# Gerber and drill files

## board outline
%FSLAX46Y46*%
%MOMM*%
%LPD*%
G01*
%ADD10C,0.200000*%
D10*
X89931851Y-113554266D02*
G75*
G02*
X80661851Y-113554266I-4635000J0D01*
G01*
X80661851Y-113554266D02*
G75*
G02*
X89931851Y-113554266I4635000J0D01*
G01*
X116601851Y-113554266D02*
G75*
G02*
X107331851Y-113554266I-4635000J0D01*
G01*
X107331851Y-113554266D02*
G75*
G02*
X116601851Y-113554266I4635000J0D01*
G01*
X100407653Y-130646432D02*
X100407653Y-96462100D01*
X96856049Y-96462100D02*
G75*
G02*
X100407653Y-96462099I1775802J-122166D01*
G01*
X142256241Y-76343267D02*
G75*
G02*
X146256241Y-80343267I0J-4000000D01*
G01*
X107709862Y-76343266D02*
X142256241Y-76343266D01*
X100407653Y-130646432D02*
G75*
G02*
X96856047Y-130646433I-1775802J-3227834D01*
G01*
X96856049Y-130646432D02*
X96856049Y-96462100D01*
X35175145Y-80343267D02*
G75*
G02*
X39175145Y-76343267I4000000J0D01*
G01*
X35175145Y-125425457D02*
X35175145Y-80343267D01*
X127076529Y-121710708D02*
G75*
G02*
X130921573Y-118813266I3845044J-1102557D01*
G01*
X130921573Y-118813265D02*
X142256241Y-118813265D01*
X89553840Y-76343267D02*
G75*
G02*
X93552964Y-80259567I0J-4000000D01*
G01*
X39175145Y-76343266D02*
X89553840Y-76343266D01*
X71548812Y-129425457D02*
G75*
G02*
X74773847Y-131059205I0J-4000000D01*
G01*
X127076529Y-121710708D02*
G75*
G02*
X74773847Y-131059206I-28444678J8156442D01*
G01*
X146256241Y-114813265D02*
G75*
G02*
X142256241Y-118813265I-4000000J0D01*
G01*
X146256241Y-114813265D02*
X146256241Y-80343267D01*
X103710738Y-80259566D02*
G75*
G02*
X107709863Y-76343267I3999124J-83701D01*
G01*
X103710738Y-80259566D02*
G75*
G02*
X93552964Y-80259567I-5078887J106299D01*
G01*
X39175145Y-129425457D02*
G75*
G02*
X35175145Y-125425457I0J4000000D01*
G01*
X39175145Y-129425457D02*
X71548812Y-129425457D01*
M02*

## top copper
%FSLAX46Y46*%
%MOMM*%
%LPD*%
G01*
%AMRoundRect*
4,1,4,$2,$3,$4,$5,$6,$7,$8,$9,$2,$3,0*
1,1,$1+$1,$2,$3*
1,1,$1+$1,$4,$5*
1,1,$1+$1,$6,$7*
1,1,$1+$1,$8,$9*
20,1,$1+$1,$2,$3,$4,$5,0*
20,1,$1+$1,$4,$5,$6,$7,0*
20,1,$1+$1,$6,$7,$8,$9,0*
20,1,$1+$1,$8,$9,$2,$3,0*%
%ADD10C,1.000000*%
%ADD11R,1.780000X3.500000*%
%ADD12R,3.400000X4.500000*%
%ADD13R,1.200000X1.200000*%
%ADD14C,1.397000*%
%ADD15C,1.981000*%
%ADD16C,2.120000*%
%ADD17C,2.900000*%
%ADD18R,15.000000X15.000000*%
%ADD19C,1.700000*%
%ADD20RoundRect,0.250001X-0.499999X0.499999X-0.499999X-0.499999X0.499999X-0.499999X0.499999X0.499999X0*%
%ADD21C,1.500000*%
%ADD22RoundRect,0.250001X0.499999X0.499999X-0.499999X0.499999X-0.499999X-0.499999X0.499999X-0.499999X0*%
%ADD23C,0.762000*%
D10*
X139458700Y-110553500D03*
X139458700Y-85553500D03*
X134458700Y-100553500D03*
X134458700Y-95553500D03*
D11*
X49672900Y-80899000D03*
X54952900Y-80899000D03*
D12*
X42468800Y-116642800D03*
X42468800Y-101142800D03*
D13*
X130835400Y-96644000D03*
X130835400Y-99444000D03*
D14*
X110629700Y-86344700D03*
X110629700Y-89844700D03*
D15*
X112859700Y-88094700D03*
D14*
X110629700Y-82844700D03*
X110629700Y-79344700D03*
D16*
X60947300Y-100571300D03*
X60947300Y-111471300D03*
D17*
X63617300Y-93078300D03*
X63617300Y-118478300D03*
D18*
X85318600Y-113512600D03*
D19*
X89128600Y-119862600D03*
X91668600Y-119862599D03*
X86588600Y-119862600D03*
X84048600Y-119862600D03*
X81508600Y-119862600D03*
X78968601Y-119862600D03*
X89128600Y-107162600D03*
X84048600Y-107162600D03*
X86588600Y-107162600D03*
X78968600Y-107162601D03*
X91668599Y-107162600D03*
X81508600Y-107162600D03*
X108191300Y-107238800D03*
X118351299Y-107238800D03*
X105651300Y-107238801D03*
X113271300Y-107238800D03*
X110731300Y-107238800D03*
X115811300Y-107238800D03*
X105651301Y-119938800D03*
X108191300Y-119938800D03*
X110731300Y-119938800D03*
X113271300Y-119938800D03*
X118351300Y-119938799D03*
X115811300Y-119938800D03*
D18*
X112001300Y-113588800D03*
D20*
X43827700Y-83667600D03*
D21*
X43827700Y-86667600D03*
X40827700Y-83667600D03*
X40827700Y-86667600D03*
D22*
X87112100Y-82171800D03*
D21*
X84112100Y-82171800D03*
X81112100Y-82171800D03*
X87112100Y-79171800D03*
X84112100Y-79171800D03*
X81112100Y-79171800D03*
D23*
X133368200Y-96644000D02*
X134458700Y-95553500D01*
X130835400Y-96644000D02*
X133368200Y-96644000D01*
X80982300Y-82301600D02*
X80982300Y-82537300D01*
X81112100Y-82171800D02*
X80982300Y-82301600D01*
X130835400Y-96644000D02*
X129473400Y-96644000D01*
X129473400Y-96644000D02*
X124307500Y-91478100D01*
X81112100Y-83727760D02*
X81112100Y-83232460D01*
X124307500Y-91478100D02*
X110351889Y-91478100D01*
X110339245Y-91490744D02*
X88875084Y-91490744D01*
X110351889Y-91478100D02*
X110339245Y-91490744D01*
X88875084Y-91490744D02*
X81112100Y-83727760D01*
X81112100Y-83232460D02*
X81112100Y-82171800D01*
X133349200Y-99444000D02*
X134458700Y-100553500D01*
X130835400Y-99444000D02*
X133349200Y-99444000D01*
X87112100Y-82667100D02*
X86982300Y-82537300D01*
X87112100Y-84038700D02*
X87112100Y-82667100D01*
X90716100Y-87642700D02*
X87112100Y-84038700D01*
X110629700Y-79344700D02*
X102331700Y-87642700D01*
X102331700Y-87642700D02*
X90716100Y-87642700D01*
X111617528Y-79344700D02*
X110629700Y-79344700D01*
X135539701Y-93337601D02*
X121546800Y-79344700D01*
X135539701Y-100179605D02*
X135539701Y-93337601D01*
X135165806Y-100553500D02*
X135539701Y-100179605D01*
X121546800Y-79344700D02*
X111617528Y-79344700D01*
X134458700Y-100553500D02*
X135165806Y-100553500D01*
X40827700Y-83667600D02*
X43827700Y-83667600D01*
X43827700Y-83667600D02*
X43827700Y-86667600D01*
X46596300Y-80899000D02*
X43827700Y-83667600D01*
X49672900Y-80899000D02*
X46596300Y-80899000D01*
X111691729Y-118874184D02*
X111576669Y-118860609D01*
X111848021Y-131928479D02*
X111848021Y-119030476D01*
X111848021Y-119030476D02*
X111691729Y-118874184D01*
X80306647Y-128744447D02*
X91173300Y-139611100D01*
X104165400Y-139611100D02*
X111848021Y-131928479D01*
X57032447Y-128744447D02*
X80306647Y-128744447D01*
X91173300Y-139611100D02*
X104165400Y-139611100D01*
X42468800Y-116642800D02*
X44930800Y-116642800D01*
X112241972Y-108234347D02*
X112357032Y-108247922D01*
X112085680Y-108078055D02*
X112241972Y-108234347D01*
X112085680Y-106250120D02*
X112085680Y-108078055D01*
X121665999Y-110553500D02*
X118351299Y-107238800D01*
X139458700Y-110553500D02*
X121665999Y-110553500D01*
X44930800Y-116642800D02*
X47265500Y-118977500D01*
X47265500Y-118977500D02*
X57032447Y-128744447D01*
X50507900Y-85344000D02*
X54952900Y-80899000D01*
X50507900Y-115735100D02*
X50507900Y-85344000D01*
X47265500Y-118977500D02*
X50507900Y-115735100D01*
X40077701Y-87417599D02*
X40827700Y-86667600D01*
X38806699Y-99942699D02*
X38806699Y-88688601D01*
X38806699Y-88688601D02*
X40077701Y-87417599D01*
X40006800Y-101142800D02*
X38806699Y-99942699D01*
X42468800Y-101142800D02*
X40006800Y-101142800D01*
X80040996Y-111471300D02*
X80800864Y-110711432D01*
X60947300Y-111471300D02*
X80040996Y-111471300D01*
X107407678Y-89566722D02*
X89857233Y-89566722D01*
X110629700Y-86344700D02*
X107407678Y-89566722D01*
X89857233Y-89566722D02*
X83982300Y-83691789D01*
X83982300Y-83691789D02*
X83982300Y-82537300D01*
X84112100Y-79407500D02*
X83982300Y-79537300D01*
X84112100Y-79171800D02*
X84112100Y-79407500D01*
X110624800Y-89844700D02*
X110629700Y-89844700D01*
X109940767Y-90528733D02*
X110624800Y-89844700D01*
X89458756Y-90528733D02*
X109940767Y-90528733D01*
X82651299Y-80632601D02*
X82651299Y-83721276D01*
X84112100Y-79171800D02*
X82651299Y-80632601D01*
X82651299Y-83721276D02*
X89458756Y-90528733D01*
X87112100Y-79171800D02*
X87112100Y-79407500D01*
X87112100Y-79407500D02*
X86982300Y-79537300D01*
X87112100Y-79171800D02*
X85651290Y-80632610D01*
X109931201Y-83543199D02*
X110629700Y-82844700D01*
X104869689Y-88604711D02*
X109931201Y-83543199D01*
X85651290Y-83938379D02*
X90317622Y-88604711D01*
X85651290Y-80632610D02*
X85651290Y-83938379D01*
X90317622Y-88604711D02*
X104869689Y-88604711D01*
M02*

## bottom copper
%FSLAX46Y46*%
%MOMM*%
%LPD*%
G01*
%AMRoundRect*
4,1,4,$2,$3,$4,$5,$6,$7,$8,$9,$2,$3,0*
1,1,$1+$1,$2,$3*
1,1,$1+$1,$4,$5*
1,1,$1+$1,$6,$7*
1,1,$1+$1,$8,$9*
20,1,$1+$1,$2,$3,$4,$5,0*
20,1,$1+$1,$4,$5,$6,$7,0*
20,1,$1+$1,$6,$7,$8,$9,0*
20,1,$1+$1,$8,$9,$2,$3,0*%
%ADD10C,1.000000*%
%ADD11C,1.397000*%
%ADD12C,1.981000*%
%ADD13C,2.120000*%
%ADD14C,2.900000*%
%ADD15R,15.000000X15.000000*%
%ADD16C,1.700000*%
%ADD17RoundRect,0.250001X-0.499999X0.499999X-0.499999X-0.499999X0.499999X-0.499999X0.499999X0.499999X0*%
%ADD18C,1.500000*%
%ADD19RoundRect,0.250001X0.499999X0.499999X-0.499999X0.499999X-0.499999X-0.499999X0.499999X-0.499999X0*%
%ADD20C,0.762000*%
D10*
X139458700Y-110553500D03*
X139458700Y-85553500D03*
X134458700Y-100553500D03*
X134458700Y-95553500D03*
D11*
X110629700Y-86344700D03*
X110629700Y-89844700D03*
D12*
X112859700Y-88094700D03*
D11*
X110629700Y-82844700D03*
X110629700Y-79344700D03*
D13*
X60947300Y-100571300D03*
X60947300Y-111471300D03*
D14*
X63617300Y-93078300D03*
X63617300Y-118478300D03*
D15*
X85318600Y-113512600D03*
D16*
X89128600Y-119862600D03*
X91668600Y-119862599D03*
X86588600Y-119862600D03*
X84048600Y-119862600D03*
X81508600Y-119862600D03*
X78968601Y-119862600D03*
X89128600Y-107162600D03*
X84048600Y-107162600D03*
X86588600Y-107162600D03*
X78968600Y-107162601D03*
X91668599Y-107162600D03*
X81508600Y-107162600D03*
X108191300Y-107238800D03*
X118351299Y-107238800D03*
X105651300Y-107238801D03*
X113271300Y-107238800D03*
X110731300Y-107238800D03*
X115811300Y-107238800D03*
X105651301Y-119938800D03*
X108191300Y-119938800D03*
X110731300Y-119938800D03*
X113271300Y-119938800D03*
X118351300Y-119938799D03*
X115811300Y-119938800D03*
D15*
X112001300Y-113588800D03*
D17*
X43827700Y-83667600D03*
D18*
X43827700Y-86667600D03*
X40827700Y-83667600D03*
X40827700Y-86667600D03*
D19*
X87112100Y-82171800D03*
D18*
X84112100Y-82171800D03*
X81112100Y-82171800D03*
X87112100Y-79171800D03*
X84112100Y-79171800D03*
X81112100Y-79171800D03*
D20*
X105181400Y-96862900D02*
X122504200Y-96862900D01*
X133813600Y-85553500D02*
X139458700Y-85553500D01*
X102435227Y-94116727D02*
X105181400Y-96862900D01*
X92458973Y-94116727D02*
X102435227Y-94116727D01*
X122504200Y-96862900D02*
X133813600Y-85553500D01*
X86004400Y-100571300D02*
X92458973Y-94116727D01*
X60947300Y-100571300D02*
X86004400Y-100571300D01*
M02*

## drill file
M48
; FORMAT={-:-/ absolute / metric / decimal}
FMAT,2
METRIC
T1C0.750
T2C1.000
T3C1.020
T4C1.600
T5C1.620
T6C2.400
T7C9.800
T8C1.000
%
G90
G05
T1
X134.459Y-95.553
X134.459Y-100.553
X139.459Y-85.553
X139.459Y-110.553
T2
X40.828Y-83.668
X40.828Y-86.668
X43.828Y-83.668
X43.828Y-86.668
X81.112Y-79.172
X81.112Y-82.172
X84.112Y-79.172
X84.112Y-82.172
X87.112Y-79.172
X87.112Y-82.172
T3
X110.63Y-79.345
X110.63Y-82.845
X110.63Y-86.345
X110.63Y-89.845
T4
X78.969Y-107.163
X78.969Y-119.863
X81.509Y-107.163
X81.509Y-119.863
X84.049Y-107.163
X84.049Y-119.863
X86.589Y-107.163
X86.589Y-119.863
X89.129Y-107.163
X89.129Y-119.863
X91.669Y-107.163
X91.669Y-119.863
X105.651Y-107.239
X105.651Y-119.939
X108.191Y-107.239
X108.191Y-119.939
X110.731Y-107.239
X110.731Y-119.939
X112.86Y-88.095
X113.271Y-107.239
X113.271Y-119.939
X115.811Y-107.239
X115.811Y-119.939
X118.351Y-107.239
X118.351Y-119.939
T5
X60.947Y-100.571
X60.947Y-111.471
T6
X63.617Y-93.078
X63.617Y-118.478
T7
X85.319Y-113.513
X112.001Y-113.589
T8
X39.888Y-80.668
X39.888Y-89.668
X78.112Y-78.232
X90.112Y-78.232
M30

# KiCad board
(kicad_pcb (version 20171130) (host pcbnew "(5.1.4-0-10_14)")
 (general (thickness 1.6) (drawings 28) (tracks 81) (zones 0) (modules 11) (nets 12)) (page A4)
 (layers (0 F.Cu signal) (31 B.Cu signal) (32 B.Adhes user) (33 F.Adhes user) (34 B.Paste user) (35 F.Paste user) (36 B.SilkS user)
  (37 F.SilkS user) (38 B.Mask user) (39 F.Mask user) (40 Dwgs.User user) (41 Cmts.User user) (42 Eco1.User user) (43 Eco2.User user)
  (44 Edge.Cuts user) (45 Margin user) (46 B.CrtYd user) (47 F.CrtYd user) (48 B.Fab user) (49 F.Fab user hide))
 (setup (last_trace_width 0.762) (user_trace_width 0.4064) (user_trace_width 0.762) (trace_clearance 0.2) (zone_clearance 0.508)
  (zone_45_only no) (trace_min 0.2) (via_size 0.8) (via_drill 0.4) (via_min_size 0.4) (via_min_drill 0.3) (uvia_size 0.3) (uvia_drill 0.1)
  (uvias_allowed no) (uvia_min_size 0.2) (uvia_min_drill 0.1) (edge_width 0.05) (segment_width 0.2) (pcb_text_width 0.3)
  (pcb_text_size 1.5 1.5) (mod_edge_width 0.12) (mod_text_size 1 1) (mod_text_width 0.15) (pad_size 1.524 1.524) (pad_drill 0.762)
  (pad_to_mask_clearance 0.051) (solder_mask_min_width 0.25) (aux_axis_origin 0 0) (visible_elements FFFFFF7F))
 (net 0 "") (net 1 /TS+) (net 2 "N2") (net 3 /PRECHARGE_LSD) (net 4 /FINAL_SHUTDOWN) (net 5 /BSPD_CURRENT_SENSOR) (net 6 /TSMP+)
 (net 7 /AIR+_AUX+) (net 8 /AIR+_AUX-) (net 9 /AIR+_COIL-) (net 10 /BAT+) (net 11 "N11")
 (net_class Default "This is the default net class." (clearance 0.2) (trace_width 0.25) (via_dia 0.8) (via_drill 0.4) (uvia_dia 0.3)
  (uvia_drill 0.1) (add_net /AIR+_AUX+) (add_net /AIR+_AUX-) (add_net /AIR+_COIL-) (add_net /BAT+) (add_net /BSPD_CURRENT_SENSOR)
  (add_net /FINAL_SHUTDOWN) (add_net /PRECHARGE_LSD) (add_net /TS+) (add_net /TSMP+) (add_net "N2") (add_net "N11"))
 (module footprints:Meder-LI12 (layer F.Cu) (at 139.4587 110.5535 90)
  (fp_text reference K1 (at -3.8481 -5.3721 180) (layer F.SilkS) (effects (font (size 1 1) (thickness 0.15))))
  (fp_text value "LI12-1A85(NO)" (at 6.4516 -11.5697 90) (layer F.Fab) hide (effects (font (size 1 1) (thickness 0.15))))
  (pad 1 thru_hole circle (at 0 0 90) (size 1 1) (drill 0.75) (layers *.Cu *.Mask) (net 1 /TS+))
  (pad 2 thru_hole circle (at 25 0 90) (size 1 1) (drill 0.75) (layers *.Cu *.Mask) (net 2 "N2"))
  (pad 3 thru_hole circle (at 10 -5 90) (size 1 1) (drill 0.75) (layers *.Cu *.Mask) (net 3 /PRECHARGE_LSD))
  (pad 4 thru_hole circle (at 15 -5 90) (size 1 1) (drill 0.75) (layers *.Cu *.Mask) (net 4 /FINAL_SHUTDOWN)))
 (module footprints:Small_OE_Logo (layer F.Cu) (at 84.9503 96.774)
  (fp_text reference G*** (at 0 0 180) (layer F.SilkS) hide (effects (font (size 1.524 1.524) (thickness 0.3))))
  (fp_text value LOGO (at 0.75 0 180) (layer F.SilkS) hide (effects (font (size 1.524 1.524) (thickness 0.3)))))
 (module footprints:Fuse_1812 (layer F.Cu) (at 54.9529 80.899 180)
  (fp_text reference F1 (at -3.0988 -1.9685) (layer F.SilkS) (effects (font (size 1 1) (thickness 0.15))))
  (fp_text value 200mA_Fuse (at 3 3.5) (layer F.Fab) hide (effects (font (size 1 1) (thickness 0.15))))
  (pad 2 smd rect (at 5.28 0 180) (size 1.78 3.5) (layers F.Cu F.Paste F.Mask) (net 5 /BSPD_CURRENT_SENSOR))
  (pad 1 smd rect (at 0 0 180) (size 1.78 3.5) (layers F.Cu F.Paste F.Mask) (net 1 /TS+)))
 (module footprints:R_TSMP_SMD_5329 (layer F.Cu) (at 42.4688 108.7628 270)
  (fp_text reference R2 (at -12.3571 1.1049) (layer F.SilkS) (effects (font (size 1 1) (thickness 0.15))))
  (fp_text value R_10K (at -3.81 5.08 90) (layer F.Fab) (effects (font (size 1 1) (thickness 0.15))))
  (pad 2 smd rect (at 7.88 0 270) (size 4.5 3.4) (layers F.Cu F.Paste F.Mask) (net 1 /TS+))
  (pad 1 smd rect (at -7.62 0 270) (size 4.5 3.4) (layers F.Cu F.Paste F.Mask) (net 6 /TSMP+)))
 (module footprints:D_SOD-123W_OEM (layer F.Cu) (at 130.8354 98.044 270)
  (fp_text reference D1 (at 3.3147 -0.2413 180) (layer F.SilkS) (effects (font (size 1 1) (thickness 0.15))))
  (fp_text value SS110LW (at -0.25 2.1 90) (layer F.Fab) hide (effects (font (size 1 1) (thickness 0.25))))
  (pad 1 smd rect (at -1.4 0 270) (size 1.2 1.2) (layers F.Cu F.Paste F.Mask) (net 4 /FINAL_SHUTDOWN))
  (pad 2 smd rect (at 1.4 0 270) (size 1.2 1.2) (layers F.Cu F.Paste F.Mask) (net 3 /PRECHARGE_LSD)))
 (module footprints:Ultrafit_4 (layer F.Cu) (at 110.6297 84.5947)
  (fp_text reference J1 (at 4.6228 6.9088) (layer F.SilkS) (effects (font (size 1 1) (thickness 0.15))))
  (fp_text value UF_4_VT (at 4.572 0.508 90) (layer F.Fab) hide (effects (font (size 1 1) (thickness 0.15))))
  (pad 2 thru_hole circle (at 0 1.75) (size 1.397 1.397) (drill 1.02) (layers *.Cu *.Mask) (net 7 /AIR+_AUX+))
  (pad 1 thru_hole circle (at 0 5.25) (size 1.397 1.397) (drill 1.02) (layers *.Cu *.Mask) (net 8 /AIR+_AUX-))
  (pad "" thru_hole circle (at 2.23 3.5) (size 1.981 1.981) (drill 1.6) (layers *.Cu *.Mask))
  (pad 3 thru_hole circle (at 0 -1.75 180) (size 1.397 1.397) (drill 1.02) (layers *.Cu *.Mask) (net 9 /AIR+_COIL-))
  (pad 4 thru_hole circle (at 0 -5.25 180) (size 1.397 1.397) (drill 1.02) (layers *.Cu *.Mask) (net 3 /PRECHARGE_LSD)))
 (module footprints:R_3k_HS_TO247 (layer F.Cu) (at 60.9473 100.5713 270)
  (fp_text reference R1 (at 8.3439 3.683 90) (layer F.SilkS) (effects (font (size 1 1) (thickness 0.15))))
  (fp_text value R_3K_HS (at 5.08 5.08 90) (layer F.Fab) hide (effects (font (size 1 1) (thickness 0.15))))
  (pad 1 thru_hole circle (at 0 0 270) (size 2.12 2.12) (drill 1.62) (layers *.Cu *.Mask) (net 2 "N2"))
  (pad 2 thru_hole circle (at 10.9 0 270) (size 2.12 2.12) (drill 1.62) (layers *.Cu *.Mask) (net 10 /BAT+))
  (pad 4 thru_hole circle (at -7.493 -2.67 270) (size 2.9 2.9) (drill 2.4) (layers *.Cu *.Mask))
  (pad 5 thru_hole circle (at 17.907 -2.67 270) (size 2.9 2.9) (drill 2.4) (layers *.Cu *.Mask)))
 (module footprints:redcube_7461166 (layer F.Cu) (at 85.3186 113.5126)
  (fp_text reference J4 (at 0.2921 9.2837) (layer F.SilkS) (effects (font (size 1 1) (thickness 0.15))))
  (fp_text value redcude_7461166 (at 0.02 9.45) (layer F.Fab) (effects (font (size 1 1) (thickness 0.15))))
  (pad 1 thru_hole rect (at 0 0) (size 15 15) (drill 9.8) (layers *.Cu *.Mask) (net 10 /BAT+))
  (pad 1 thru_hole circle (at 3.81 6.35) (size 1.7 1.7) (drill 1.6) (layers *.Cu *.Mask) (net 10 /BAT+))
  (pad 1 thru_hole circle (at 6.35 6.349999) (size 1.7 1.7) (drill 1.6) (layers *.Cu *.Mask) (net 10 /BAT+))
  (pad 1 thru_hole circle (at 1.27 6.35) (size 1.7 1.7) (drill 1.6) (layers *.Cu *.Mask) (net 10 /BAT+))
  (pad 1 thru_hole circle (at -1.27 6.35) (size 1.7 1.7) (drill 1.6) (layers *.Cu *.Mask) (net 10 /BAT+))
  (pad 1 thru_hole circle (at -3.81 6.35) (size 1.7 1.7) (drill 1.6) (layers *.Cu *.Mask) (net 10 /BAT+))
  (pad 1 thru_hole circle (at -6.349999 6.35) (size 1.7 1.7) (drill 1.6) (layers *.Cu *.Mask) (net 10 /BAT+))
  (pad 1 thru_hole circle (at 3.81 -6.35) (size 1.7 1.7) (drill 1.6) (layers *.Cu *.Mask) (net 10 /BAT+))
  (pad 1 thru_hole circle (at -1.27 -6.35) (size 1.7 1.7) (drill 1.6) (layers *.Cu *.Mask) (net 10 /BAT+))
  (pad 1 thru_hole circle (at 1.27 -6.35) (size 1.7 1.7) (drill 1.6) (layers *.Cu *.Mask) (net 10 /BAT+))
  (pad 1 thru_hole circle (at -6.35 -6.349999) (size 1.7 1.7) (drill 1.6) (layers *.Cu *.Mask) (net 10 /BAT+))
  (pad 1 thru_hole circle (at 6.349999 -6.35) (size 1.7 1.7) (drill 1.6) (layers *.Cu *.Mask) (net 10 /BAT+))
  (pad 1 thru_hole circle (at -3.81 -6.35) (size 1.7 1.7) (drill 1.6) (layers *.Cu *.Mask) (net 10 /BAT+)))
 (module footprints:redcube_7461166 (layer F.Cu) (at 112.0013 113.5888)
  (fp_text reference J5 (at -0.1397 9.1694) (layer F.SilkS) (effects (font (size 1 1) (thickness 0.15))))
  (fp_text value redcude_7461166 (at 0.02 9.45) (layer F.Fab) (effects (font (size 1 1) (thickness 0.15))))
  (pad 1 thru_hole circle (at -3.81 -6.35) (size 1.7 1.7) (drill 1.6) (layers *.Cu *.Mask) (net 1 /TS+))
  (pad 1 thru_hole circle (at 6.349999 -6.35) (size 1.7 1.7) (drill 1.6) (layers *.Cu *.Mask) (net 1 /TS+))
  (pad 1 thru_hole circle (at -6.35 -6.349999) (size 1.7 1.7) (drill 1.6) (layers *.Cu *.Mask) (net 1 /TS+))
  (pad 1 thru_hole circle (at 1.27 -6.35) (size 1.7 1.7) (drill 1.6) (layers *.Cu *.Mask) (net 1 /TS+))
  (pad 1 thru_hole circle (at -1.27 -6.35) (size 1.7 1.7) (drill 1.6) (layers *.Cu *.Mask) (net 1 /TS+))
  (pad 1 thru_hole circle (at 3.81 -6.35) (size 1.7 1.7) (drill 1.6) (layers *.Cu *.Mask) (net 1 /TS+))
  (pad 1 thru_hole circle (at -6.349999 6.35) (size 1.7 1.7) (drill 1.6) (layers *.Cu *.Mask) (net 1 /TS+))
  (pad 1 thru_hole circle (at -3.81 6.35) (size 1.7 1.7) (drill 1.6) (layers *.Cu *.Mask) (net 1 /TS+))
  (pad 1 thru_hole circle (at -1.27 6.35) (size 1.7 1.7) (drill 1.6) (layers *.Cu *.Mask) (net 1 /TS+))
  (pad 1 thru_hole circle (at 1.27 6.35) (size 1.7 1.7) (drill 1.6) (layers *.Cu *.Mask) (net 1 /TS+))
  (pad 1 thru_hole circle (at 6.35 6.349999) (size 1.7 1.7) (drill 1.6) (layers *.Cu *.Mask) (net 1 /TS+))
  (pad 1 thru_hole circle (at 3.81 6.35) (size 1.7 1.7) (drill 1.6) (layers *.Cu *.Mask) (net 1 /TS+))
  (pad 1 thru_hole rect (at 0 0) (size 15 15) (drill 9.8) (layers *.Cu *.Mask) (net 1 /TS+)))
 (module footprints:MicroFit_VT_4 (layer F.Cu) (at 43.8277 83.6676 270)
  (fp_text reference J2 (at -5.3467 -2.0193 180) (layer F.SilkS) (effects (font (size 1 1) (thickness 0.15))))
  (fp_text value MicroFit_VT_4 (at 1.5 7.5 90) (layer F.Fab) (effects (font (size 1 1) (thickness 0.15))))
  (pad "" np_thru_hole circle (at -3 3.94 270) (size 1 1) (drill 1) (layers *.Cu *.Mask))
  (pad "" np_thru_hole circle (at 6 3.94 270) (size 1 1) (drill 1) (layers *.Cu *.Mask))
  (pad 1 thru_hole roundrect (at 0 0 270) (size 1.5 1.5) (drill 1) (layers *.Cu *.Mask) (roundrect_rratio 0.166667)
   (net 5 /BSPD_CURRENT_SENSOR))
  (pad 2 thru_hole circle (at 3 0 270) (size 1.5 1.5) (drill 1) (layers *.Cu *.Mask) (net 5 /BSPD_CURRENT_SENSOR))
  (pad 3 thru_hole circle (at 0 3 270) (size 1.5 1.5) (drill 1) (layers *.Cu *.Mask) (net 5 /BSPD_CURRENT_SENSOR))
  (pad 4 thru_hole circle (at 3 3 270) (size 1.5 1.5) (drill 1) (layers *.Cu *.Mask) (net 6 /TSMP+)))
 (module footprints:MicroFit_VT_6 (layer F.Cu) (at 87.1121 82.1718 180)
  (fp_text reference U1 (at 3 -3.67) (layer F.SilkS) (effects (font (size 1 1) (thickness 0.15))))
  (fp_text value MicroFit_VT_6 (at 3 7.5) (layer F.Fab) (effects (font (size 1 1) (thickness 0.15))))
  (pad "" np_thru_hole circle (at -3 3.94 180) (size 1 1) (drill 1) (layers *.Cu *.Mask))
  (pad "" np_thru_hole circle (at 9 3.94 180) (size 1 1) (drill 1) (layers *.Cu *.Mask))
  (pad 1 thru_hole roundrect (at 0 0 180) (size 1.5 1.5) (drill 1) (layers *.Cu *.Mask) (roundrect_rratio 0.166667) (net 3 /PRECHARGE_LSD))
  (pad 2 thru_hole circle (at 3 0 180) (size 1.5 1.5) (drill 1) (layers *.Cu *.Mask) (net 7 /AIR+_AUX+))
  (pad 3 thru_hole circle (at 6 0 180) (size 1.5 1.5) (drill 1) (layers *.Cu *.Mask) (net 4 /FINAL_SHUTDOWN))
  (pad 4 thru_hole circle (at 0 3 180) (size 1.5 1.5) (drill 1) (layers *.Cu *.Mask) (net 9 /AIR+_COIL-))
  (pad 5 thru_hole circle (at 3 3 180) (size 1.5 1.5) (drill 1) (layers *.Cu *.Mask) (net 8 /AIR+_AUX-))
  (pad 6 thru_hole circle (at 6 3 180) (size 1.5 1.5) (drill 1) (layers *.Cu *.Mask) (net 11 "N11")))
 (gr_circle (center 85.296851 113.554266) (end 89.931851 113.554266) (layer Edge.Cuts) (width 0.2))
 (gr_circle (center 111.966851 113.554266) (end 116.601851 113.554266) (layer Edge.Cuts) (width 0.2))
 (gr_line (start 100.407653 130.646432) (end 100.407653 96.4621) (layer Edge.Cuts) (width 0.2))
 (gr_arc (start 98.631851 96.584266) (end 96.856049 96.4621) (angle 172.1290524) (layer Edge.Cuts) (width 0.2))
 (gr_arc (start 142.256241 80.343267) (end 142.256241 76.343267) (angle 90) (layer Edge.Cuts) (width 0.2))
 (gr_line (start 107.709862 76.343266) (end 142.256241 76.343266) (layer Edge.Cuts) (width 0.2))
 (gr_arc (start 98.631851 133.874266) (end 100.407653 130.646432) (angle 302.3649367) (layer Edge.Cuts) (width 0.2))
 (gr_line (start 96.856049 130.646432) (end 96.856049 96.4621) (layer Edge.Cuts) (width 0.2))
 (gr_arc (start 39.175145 80.343267) (end 35.175145 80.343267) (angle 90) (layer Edge.Cuts) (width 0.2))
 (gr_line (start 35.175145 125.425457) (end 35.175145 80.343267) (layer Edge.Cuts) (width 0.2))
 (gr_arc (start 130.921573 122.813265) (end 127.076529 121.710708) (angle 73.99988382) (layer Edge.Cuts) (width 0.2))
 (gr_line (start 130.921573 118.813265) (end 142.256241 118.813265) (layer Edge.Cuts) (width 0.2))
 (gr_arc (start 89.55384 80.343267) (end 89.55384 76.343267) (angle 88.80099199) (layer Edge.Cuts) (width 0.2))
 (gr_line (start 39.175145 76.343266) (end 89.55384 76.343266) (layer Edge.Cuts) (width 0.2))
 (gr_arc (start 71.548812 133.425457) (end 71.548812 129.425457) (angle 53.73200085) (layer Edge.Cuts) (width 0.2))
 (gr_arc (start 98.631851 113.554266) (end 127.076529 121.710708) (angle 127.7318847) (layer Edge.Cuts) (width 0.2))
 (gr_arc (start 142.256241 114.813265) (end 146.256241 114.813265) (angle 90) (layer Edge.Cuts) (width 0.2))
 (gr_line (start 146.256241 114.813265) (end 146.256241 80.343267) (layer Edge.Cuts) (width 0.2))
 (gr_arc (start 107.709862 80.343267) (end 103.710738 80.259566) (angle 88.80099199) (layer Edge.Cuts) (width 0.2))
 (gr_arc (start 98.631851 80.153267) (end 103.710738 80.259566) (angle 177.601984) (layer Edge.Cuts) (width 0.2))
 (gr_arc (start 39.175145 125.425457) (end 39.175145 129.425457) (angle 90) (layer Edge.Cuts) (width 0.2))
 (gr_line (start 39.175145 129.425457) (end 71.548812 129.425457) (layer Edge.Cuts) (width 0.2))
 (segment (start 133.3682 96.644) (end 134.4587 95.5535) (width 0.762) (layer F.Cu) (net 4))
 (segment (start 130.8354 96.644) (end 133.3682 96.644) (width 0.762) (layer F.Cu) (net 4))
 (segment (start 80.9823 82.3016) (end 80.9823 82.5373) (width 0.762) (layer F.Cu) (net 4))
 (segment (start 81.1121 82.1718) (end 80.9823 82.3016) (width 0.762) (layer F.Cu) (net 4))
 (segment (start 130.8354 96.644) (end 129.4734 96.644) (width 0.762) (layer F.Cu) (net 4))
 (segment (start 129.4734 96.644) (end 124.3075 91.4781) (width 0.762) (layer F.Cu) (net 4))
 (segment (start 81.1121 83.72776) (end 81.1121 83.23246) (width 0.762) (layer F.Cu) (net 4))
 (segment (start 124.3075 91.4781) (end 110.351889 91.4781) (width 0.762) (layer F.Cu) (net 4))
 (segment (start 110.339245 91.490744) (end 88.875084 91.490744) (width 0.762) (layer F.Cu) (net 4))
 (segment (start 110.351889 91.4781) (end 110.339245 91.490744) (width 0.762) (layer F.Cu) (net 4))
 (segment (start 88.875084 91.490744) (end 81.1121 83.72776) (width 0.762) (layer F.Cu) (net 4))
 (segment (start 81.1121 83.23246) (end 81.1121 82.1718) (width 0.762) (layer F.Cu) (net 4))
 (segment (start 133.3492 99.444) (end 134.4587 100.5535) (width 0.762) (layer F.Cu) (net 3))
 (segment (start 130.8354 99.444) (end 133.3492 99.444) (width 0.762) (layer F.Cu) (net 3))
 (segment (start 87.1121 82.6671) (end 86.9823 82.5373) (width 0.762) (layer F.Cu) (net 3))
 (segment (start 87.1121 84.0387) (end 87.1121 82.6671) (width 0.762) (layer F.Cu) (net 3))
 (segment (start 90.7161 87.6427) (end 87.1121 84.0387) (width 0.762) (layer F.Cu) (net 3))
 (segment (start 110.6297 79.3447) (end 102.3317 87.6427) (width 0.762) (layer F.Cu) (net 3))
 (segment (start 102.3317 87.6427) (end 90.7161 87.6427) (width 0.762) (layer F.Cu) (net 3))
 (segment (start 111.617528 79.3447) (end 110.6297 79.3447) (width 0.762) (layer F.Cu) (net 3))
 (segment (start 135.539701 93.337601) (end 121.5468 79.3447) (width 0.762) (layer F.Cu) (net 3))
 (segment (start 135.539701 100.179605) (end 135.539701 93.337601) (width 0.762) (layer F.Cu) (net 3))
 (segment (start 135.165806 100.5535) (end 135.539701 100.179605) (width 0.762) (layer F.Cu) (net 3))
 (segment (start 121.5468 79.3447) (end 111.617528 79.3447) (width 0.762) (layer F.Cu) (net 3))
 (segment (start 134.4587 100.5535) (end 135.165806 100.5535) (width 0.762) (layer F.Cu) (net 3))
 (segment (start 40.8277 83.6676) (end 43.8277 83.6676) (width 0.762) (layer F.Cu) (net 5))
 (segment (start 43.8277 83.6676) (end 43.8277 86.6676) (width 0.762) (layer F.Cu) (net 5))
 (segment (start 46.5963 80.899) (end 43.8277 83.6676) (width 0.762) (layer F.Cu) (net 5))
 (segment (start 49.6729 80.899) (end 46.5963 80.899) (width 0.762) (layer F.Cu) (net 5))
 (segment (start 111.691729 118.874184) (end 111.576669 118.860609) (width 0.762) (layer F.Cu) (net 1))
 (segment (start 111.848021 131.928479) (end 111.848021 119.030476) (width 0.762) (layer F.Cu) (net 1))
 (segment (start 111.848021 119.030476) (end 111.691729 118.874184) (width 0.762) (layer F.Cu) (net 1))
 (segment (start 80.306647 128.744447) (end 91.1733 139.6111) (width 0.762) (layer F.Cu) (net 1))
 (segment (start 104.1654 139.6111) (end 111.848021 131.928479) (width 0.762) (layer F.Cu) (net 1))
 (segment (start 57.032447 128.744447) (end 80.306647 128.744447) (width 0.762) (layer F.Cu) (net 1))
 (segment (start 91.1733 139.6111) (end 104.1654 139.6111) (width 0.762) (layer F.Cu) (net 1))
 (segment (start 42.4688 116.6428) (end 44.9308 116.6428) (width 0.762) (layer F.Cu) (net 1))
 (segment (start 112.241972 108.234347) (end 112.357032 108.247922) (width 0.762) (layer F.Cu) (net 1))
 (segment (start 112.08568 108.078055) (end 112.241972 108.234347) (width 0.762) (layer F.Cu) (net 1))
 (segment (start 112.08568 106.25012) (end 112.08568 108.078055) (width 0.762) (layer F.Cu) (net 1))
 (segment (start 121.665999 110.5535) (end 118.351299 107.2388) (width 0.762) (layer F.Cu) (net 1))
 (segment (start 139.4587 110.5535) (end 121.665999 110.5535) (width 0.762) (layer F.Cu) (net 1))
 (segment (start 44.9308 116.6428) (end 47.2655 118.9775) (width 0.762) (layer F.Cu) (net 1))
 (segment (start 47.2655 118.9775) (end 57.032447 128.744447) (width 0.762) (layer F.Cu) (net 1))
 (segment (start 50.5079 85.344) (end 54.9529 80.899) (width 0.762) (layer F.Cu) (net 1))
 (segment (start 50.5079 115.7351) (end 50.5079 85.344) (width 0.762) (layer F.Cu) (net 1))
 (segment (start 47.2655 118.9775) (end 50.5079 115.7351) (width 0.762) (layer F.Cu) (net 1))
 (segment (start 40.077701 87.417599) (end 40.8277 86.6676) (width 0.762) (layer F.Cu) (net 6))
 (segment (start 38.806699 99.942699) (end 38.806699 88.688601) (width 0.762) (layer F.Cu) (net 6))
 (segment (start 38.806699 88.688601) (end 40.077701 87.417599) (width 0.762) (layer F.Cu) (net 6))
 (segment (start 40.0068 101.1428) (end 38.806699 99.942699) (width 0.762) (layer F.Cu) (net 6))
 (segment (start 42.4688 101.1428) (end 40.0068 101.1428) (width 0.762) (layer F.Cu) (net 6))
 (segment (start 80.040996 111.4713) (end 80.800864 110.711432) (width 0.762) (layer F.Cu) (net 10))
 (segment (start 60.9473 111.4713) (end 80.040996 111.4713) (width 0.762) (layer F.Cu) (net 10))
 (segment (start 105.1814 96.8629) (end 122.5042 96.8629) (width 0.762) (layer B.Cu) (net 2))
 (segment (start 133.8136 85.5535) (end 139.4587 85.5535) (width 0.762) (layer B.Cu) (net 2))
 (segment (start 102.435227 94.116727) (end 105.1814 96.8629) (width 0.762) (layer B.Cu) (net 2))
 (segment (start 92.458973 94.116727) (end 102.435227 94.116727) (width 0.762) (layer B.Cu) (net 2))
 (segment (start 122.5042 96.8629) (end 133.8136 85.5535) (width 0.762) (layer B.Cu) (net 2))
 (segment (start 86.0044 100.5713) (end 92.458973 94.116727) (width 0.762) (layer B.Cu) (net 2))
 (segment (start 60.9473 100.5713) (end 86.0044 100.5713) (width 0.762) (layer B.Cu) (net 2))
 (segment (start 107.407678 89.566722) (end 89.857233 89.566722) (width 0.762) (layer F.Cu) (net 7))
 (segment (start 110.6297 86.3447) (end 107.407678 89.566722) (width 0.762) (layer F.Cu) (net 7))
 (segment (start 89.857233 89.566722) (end 83.9823 83.691789) (width 0.762) (layer F.Cu) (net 7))
 (segment (start 83.9823 83.691789) (end 83.9823 82.5373) (width 0.762) (layer F.Cu) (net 7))
 (segment (start 84.1121 79.4075) (end 83.9823 79.5373) (width 0.762) (layer F.Cu) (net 8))
 (segment (start 84.1121 79.1718) (end 84.1121 79.4075) (width 0.762) (layer F.Cu) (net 8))
 (segment (start 110.6248 89.8447) (end 110.6297 89.8447) (width 0.762) (layer F.Cu) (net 8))
 (segment (start 109.940767 90.528733) (end 110.6248 89.8447) (width 0.762) (layer F.Cu) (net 8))
 (segment (start 89.458756 90.528733) (end 109.940767 90.528733) (width 0.762) (layer F.Cu) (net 8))
 (segment (start 82.651299 80.632601) (end 82.651299 83.721276) (width 0.762) (layer F.Cu) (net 8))
 (segment (start 84.1121 79.1718) (end 82.651299 80.632601) (width 0.762) (layer F.Cu) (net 8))
 (segment (start 82.651299 83.721276) (end 89.458756 90.528733) (width 0.762) (layer F.Cu) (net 8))
 (segment (start 87.1121 79.1718) (end 87.1121 79.4075) (width 0.762) (layer F.Cu) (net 9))
 (segment (start 87.1121 79.4075) (end 86.9823 79.5373) (width 0.762) (layer F.Cu) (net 9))
 (segment (start 87.1121 79.1718) (end 85.65129 80.63261) (width 0.762) (layer F.Cu) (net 9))
 (segment (start 109.931201 83.543199) (end 110.6297 82.8447) (width 0.762) (layer F.Cu) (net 9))
 (segment (start 104.869689 88.604711) (end 109.931201 83.543199) (width 0.762) (layer F.Cu) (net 9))
 (segment (start 85.65129 83.938379) (end 90.317622 88.604711) (width 0.762) (layer F.Cu) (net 9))
 (segment (start 85.65129 80.63261) (end 85.65129 83.938379) (width 0.762) (layer F.Cu) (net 9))
 (segment (start 90.317622 88.604711) (end 104.869689 88.604711) (width 0.762) (layer F.Cu) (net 9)))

